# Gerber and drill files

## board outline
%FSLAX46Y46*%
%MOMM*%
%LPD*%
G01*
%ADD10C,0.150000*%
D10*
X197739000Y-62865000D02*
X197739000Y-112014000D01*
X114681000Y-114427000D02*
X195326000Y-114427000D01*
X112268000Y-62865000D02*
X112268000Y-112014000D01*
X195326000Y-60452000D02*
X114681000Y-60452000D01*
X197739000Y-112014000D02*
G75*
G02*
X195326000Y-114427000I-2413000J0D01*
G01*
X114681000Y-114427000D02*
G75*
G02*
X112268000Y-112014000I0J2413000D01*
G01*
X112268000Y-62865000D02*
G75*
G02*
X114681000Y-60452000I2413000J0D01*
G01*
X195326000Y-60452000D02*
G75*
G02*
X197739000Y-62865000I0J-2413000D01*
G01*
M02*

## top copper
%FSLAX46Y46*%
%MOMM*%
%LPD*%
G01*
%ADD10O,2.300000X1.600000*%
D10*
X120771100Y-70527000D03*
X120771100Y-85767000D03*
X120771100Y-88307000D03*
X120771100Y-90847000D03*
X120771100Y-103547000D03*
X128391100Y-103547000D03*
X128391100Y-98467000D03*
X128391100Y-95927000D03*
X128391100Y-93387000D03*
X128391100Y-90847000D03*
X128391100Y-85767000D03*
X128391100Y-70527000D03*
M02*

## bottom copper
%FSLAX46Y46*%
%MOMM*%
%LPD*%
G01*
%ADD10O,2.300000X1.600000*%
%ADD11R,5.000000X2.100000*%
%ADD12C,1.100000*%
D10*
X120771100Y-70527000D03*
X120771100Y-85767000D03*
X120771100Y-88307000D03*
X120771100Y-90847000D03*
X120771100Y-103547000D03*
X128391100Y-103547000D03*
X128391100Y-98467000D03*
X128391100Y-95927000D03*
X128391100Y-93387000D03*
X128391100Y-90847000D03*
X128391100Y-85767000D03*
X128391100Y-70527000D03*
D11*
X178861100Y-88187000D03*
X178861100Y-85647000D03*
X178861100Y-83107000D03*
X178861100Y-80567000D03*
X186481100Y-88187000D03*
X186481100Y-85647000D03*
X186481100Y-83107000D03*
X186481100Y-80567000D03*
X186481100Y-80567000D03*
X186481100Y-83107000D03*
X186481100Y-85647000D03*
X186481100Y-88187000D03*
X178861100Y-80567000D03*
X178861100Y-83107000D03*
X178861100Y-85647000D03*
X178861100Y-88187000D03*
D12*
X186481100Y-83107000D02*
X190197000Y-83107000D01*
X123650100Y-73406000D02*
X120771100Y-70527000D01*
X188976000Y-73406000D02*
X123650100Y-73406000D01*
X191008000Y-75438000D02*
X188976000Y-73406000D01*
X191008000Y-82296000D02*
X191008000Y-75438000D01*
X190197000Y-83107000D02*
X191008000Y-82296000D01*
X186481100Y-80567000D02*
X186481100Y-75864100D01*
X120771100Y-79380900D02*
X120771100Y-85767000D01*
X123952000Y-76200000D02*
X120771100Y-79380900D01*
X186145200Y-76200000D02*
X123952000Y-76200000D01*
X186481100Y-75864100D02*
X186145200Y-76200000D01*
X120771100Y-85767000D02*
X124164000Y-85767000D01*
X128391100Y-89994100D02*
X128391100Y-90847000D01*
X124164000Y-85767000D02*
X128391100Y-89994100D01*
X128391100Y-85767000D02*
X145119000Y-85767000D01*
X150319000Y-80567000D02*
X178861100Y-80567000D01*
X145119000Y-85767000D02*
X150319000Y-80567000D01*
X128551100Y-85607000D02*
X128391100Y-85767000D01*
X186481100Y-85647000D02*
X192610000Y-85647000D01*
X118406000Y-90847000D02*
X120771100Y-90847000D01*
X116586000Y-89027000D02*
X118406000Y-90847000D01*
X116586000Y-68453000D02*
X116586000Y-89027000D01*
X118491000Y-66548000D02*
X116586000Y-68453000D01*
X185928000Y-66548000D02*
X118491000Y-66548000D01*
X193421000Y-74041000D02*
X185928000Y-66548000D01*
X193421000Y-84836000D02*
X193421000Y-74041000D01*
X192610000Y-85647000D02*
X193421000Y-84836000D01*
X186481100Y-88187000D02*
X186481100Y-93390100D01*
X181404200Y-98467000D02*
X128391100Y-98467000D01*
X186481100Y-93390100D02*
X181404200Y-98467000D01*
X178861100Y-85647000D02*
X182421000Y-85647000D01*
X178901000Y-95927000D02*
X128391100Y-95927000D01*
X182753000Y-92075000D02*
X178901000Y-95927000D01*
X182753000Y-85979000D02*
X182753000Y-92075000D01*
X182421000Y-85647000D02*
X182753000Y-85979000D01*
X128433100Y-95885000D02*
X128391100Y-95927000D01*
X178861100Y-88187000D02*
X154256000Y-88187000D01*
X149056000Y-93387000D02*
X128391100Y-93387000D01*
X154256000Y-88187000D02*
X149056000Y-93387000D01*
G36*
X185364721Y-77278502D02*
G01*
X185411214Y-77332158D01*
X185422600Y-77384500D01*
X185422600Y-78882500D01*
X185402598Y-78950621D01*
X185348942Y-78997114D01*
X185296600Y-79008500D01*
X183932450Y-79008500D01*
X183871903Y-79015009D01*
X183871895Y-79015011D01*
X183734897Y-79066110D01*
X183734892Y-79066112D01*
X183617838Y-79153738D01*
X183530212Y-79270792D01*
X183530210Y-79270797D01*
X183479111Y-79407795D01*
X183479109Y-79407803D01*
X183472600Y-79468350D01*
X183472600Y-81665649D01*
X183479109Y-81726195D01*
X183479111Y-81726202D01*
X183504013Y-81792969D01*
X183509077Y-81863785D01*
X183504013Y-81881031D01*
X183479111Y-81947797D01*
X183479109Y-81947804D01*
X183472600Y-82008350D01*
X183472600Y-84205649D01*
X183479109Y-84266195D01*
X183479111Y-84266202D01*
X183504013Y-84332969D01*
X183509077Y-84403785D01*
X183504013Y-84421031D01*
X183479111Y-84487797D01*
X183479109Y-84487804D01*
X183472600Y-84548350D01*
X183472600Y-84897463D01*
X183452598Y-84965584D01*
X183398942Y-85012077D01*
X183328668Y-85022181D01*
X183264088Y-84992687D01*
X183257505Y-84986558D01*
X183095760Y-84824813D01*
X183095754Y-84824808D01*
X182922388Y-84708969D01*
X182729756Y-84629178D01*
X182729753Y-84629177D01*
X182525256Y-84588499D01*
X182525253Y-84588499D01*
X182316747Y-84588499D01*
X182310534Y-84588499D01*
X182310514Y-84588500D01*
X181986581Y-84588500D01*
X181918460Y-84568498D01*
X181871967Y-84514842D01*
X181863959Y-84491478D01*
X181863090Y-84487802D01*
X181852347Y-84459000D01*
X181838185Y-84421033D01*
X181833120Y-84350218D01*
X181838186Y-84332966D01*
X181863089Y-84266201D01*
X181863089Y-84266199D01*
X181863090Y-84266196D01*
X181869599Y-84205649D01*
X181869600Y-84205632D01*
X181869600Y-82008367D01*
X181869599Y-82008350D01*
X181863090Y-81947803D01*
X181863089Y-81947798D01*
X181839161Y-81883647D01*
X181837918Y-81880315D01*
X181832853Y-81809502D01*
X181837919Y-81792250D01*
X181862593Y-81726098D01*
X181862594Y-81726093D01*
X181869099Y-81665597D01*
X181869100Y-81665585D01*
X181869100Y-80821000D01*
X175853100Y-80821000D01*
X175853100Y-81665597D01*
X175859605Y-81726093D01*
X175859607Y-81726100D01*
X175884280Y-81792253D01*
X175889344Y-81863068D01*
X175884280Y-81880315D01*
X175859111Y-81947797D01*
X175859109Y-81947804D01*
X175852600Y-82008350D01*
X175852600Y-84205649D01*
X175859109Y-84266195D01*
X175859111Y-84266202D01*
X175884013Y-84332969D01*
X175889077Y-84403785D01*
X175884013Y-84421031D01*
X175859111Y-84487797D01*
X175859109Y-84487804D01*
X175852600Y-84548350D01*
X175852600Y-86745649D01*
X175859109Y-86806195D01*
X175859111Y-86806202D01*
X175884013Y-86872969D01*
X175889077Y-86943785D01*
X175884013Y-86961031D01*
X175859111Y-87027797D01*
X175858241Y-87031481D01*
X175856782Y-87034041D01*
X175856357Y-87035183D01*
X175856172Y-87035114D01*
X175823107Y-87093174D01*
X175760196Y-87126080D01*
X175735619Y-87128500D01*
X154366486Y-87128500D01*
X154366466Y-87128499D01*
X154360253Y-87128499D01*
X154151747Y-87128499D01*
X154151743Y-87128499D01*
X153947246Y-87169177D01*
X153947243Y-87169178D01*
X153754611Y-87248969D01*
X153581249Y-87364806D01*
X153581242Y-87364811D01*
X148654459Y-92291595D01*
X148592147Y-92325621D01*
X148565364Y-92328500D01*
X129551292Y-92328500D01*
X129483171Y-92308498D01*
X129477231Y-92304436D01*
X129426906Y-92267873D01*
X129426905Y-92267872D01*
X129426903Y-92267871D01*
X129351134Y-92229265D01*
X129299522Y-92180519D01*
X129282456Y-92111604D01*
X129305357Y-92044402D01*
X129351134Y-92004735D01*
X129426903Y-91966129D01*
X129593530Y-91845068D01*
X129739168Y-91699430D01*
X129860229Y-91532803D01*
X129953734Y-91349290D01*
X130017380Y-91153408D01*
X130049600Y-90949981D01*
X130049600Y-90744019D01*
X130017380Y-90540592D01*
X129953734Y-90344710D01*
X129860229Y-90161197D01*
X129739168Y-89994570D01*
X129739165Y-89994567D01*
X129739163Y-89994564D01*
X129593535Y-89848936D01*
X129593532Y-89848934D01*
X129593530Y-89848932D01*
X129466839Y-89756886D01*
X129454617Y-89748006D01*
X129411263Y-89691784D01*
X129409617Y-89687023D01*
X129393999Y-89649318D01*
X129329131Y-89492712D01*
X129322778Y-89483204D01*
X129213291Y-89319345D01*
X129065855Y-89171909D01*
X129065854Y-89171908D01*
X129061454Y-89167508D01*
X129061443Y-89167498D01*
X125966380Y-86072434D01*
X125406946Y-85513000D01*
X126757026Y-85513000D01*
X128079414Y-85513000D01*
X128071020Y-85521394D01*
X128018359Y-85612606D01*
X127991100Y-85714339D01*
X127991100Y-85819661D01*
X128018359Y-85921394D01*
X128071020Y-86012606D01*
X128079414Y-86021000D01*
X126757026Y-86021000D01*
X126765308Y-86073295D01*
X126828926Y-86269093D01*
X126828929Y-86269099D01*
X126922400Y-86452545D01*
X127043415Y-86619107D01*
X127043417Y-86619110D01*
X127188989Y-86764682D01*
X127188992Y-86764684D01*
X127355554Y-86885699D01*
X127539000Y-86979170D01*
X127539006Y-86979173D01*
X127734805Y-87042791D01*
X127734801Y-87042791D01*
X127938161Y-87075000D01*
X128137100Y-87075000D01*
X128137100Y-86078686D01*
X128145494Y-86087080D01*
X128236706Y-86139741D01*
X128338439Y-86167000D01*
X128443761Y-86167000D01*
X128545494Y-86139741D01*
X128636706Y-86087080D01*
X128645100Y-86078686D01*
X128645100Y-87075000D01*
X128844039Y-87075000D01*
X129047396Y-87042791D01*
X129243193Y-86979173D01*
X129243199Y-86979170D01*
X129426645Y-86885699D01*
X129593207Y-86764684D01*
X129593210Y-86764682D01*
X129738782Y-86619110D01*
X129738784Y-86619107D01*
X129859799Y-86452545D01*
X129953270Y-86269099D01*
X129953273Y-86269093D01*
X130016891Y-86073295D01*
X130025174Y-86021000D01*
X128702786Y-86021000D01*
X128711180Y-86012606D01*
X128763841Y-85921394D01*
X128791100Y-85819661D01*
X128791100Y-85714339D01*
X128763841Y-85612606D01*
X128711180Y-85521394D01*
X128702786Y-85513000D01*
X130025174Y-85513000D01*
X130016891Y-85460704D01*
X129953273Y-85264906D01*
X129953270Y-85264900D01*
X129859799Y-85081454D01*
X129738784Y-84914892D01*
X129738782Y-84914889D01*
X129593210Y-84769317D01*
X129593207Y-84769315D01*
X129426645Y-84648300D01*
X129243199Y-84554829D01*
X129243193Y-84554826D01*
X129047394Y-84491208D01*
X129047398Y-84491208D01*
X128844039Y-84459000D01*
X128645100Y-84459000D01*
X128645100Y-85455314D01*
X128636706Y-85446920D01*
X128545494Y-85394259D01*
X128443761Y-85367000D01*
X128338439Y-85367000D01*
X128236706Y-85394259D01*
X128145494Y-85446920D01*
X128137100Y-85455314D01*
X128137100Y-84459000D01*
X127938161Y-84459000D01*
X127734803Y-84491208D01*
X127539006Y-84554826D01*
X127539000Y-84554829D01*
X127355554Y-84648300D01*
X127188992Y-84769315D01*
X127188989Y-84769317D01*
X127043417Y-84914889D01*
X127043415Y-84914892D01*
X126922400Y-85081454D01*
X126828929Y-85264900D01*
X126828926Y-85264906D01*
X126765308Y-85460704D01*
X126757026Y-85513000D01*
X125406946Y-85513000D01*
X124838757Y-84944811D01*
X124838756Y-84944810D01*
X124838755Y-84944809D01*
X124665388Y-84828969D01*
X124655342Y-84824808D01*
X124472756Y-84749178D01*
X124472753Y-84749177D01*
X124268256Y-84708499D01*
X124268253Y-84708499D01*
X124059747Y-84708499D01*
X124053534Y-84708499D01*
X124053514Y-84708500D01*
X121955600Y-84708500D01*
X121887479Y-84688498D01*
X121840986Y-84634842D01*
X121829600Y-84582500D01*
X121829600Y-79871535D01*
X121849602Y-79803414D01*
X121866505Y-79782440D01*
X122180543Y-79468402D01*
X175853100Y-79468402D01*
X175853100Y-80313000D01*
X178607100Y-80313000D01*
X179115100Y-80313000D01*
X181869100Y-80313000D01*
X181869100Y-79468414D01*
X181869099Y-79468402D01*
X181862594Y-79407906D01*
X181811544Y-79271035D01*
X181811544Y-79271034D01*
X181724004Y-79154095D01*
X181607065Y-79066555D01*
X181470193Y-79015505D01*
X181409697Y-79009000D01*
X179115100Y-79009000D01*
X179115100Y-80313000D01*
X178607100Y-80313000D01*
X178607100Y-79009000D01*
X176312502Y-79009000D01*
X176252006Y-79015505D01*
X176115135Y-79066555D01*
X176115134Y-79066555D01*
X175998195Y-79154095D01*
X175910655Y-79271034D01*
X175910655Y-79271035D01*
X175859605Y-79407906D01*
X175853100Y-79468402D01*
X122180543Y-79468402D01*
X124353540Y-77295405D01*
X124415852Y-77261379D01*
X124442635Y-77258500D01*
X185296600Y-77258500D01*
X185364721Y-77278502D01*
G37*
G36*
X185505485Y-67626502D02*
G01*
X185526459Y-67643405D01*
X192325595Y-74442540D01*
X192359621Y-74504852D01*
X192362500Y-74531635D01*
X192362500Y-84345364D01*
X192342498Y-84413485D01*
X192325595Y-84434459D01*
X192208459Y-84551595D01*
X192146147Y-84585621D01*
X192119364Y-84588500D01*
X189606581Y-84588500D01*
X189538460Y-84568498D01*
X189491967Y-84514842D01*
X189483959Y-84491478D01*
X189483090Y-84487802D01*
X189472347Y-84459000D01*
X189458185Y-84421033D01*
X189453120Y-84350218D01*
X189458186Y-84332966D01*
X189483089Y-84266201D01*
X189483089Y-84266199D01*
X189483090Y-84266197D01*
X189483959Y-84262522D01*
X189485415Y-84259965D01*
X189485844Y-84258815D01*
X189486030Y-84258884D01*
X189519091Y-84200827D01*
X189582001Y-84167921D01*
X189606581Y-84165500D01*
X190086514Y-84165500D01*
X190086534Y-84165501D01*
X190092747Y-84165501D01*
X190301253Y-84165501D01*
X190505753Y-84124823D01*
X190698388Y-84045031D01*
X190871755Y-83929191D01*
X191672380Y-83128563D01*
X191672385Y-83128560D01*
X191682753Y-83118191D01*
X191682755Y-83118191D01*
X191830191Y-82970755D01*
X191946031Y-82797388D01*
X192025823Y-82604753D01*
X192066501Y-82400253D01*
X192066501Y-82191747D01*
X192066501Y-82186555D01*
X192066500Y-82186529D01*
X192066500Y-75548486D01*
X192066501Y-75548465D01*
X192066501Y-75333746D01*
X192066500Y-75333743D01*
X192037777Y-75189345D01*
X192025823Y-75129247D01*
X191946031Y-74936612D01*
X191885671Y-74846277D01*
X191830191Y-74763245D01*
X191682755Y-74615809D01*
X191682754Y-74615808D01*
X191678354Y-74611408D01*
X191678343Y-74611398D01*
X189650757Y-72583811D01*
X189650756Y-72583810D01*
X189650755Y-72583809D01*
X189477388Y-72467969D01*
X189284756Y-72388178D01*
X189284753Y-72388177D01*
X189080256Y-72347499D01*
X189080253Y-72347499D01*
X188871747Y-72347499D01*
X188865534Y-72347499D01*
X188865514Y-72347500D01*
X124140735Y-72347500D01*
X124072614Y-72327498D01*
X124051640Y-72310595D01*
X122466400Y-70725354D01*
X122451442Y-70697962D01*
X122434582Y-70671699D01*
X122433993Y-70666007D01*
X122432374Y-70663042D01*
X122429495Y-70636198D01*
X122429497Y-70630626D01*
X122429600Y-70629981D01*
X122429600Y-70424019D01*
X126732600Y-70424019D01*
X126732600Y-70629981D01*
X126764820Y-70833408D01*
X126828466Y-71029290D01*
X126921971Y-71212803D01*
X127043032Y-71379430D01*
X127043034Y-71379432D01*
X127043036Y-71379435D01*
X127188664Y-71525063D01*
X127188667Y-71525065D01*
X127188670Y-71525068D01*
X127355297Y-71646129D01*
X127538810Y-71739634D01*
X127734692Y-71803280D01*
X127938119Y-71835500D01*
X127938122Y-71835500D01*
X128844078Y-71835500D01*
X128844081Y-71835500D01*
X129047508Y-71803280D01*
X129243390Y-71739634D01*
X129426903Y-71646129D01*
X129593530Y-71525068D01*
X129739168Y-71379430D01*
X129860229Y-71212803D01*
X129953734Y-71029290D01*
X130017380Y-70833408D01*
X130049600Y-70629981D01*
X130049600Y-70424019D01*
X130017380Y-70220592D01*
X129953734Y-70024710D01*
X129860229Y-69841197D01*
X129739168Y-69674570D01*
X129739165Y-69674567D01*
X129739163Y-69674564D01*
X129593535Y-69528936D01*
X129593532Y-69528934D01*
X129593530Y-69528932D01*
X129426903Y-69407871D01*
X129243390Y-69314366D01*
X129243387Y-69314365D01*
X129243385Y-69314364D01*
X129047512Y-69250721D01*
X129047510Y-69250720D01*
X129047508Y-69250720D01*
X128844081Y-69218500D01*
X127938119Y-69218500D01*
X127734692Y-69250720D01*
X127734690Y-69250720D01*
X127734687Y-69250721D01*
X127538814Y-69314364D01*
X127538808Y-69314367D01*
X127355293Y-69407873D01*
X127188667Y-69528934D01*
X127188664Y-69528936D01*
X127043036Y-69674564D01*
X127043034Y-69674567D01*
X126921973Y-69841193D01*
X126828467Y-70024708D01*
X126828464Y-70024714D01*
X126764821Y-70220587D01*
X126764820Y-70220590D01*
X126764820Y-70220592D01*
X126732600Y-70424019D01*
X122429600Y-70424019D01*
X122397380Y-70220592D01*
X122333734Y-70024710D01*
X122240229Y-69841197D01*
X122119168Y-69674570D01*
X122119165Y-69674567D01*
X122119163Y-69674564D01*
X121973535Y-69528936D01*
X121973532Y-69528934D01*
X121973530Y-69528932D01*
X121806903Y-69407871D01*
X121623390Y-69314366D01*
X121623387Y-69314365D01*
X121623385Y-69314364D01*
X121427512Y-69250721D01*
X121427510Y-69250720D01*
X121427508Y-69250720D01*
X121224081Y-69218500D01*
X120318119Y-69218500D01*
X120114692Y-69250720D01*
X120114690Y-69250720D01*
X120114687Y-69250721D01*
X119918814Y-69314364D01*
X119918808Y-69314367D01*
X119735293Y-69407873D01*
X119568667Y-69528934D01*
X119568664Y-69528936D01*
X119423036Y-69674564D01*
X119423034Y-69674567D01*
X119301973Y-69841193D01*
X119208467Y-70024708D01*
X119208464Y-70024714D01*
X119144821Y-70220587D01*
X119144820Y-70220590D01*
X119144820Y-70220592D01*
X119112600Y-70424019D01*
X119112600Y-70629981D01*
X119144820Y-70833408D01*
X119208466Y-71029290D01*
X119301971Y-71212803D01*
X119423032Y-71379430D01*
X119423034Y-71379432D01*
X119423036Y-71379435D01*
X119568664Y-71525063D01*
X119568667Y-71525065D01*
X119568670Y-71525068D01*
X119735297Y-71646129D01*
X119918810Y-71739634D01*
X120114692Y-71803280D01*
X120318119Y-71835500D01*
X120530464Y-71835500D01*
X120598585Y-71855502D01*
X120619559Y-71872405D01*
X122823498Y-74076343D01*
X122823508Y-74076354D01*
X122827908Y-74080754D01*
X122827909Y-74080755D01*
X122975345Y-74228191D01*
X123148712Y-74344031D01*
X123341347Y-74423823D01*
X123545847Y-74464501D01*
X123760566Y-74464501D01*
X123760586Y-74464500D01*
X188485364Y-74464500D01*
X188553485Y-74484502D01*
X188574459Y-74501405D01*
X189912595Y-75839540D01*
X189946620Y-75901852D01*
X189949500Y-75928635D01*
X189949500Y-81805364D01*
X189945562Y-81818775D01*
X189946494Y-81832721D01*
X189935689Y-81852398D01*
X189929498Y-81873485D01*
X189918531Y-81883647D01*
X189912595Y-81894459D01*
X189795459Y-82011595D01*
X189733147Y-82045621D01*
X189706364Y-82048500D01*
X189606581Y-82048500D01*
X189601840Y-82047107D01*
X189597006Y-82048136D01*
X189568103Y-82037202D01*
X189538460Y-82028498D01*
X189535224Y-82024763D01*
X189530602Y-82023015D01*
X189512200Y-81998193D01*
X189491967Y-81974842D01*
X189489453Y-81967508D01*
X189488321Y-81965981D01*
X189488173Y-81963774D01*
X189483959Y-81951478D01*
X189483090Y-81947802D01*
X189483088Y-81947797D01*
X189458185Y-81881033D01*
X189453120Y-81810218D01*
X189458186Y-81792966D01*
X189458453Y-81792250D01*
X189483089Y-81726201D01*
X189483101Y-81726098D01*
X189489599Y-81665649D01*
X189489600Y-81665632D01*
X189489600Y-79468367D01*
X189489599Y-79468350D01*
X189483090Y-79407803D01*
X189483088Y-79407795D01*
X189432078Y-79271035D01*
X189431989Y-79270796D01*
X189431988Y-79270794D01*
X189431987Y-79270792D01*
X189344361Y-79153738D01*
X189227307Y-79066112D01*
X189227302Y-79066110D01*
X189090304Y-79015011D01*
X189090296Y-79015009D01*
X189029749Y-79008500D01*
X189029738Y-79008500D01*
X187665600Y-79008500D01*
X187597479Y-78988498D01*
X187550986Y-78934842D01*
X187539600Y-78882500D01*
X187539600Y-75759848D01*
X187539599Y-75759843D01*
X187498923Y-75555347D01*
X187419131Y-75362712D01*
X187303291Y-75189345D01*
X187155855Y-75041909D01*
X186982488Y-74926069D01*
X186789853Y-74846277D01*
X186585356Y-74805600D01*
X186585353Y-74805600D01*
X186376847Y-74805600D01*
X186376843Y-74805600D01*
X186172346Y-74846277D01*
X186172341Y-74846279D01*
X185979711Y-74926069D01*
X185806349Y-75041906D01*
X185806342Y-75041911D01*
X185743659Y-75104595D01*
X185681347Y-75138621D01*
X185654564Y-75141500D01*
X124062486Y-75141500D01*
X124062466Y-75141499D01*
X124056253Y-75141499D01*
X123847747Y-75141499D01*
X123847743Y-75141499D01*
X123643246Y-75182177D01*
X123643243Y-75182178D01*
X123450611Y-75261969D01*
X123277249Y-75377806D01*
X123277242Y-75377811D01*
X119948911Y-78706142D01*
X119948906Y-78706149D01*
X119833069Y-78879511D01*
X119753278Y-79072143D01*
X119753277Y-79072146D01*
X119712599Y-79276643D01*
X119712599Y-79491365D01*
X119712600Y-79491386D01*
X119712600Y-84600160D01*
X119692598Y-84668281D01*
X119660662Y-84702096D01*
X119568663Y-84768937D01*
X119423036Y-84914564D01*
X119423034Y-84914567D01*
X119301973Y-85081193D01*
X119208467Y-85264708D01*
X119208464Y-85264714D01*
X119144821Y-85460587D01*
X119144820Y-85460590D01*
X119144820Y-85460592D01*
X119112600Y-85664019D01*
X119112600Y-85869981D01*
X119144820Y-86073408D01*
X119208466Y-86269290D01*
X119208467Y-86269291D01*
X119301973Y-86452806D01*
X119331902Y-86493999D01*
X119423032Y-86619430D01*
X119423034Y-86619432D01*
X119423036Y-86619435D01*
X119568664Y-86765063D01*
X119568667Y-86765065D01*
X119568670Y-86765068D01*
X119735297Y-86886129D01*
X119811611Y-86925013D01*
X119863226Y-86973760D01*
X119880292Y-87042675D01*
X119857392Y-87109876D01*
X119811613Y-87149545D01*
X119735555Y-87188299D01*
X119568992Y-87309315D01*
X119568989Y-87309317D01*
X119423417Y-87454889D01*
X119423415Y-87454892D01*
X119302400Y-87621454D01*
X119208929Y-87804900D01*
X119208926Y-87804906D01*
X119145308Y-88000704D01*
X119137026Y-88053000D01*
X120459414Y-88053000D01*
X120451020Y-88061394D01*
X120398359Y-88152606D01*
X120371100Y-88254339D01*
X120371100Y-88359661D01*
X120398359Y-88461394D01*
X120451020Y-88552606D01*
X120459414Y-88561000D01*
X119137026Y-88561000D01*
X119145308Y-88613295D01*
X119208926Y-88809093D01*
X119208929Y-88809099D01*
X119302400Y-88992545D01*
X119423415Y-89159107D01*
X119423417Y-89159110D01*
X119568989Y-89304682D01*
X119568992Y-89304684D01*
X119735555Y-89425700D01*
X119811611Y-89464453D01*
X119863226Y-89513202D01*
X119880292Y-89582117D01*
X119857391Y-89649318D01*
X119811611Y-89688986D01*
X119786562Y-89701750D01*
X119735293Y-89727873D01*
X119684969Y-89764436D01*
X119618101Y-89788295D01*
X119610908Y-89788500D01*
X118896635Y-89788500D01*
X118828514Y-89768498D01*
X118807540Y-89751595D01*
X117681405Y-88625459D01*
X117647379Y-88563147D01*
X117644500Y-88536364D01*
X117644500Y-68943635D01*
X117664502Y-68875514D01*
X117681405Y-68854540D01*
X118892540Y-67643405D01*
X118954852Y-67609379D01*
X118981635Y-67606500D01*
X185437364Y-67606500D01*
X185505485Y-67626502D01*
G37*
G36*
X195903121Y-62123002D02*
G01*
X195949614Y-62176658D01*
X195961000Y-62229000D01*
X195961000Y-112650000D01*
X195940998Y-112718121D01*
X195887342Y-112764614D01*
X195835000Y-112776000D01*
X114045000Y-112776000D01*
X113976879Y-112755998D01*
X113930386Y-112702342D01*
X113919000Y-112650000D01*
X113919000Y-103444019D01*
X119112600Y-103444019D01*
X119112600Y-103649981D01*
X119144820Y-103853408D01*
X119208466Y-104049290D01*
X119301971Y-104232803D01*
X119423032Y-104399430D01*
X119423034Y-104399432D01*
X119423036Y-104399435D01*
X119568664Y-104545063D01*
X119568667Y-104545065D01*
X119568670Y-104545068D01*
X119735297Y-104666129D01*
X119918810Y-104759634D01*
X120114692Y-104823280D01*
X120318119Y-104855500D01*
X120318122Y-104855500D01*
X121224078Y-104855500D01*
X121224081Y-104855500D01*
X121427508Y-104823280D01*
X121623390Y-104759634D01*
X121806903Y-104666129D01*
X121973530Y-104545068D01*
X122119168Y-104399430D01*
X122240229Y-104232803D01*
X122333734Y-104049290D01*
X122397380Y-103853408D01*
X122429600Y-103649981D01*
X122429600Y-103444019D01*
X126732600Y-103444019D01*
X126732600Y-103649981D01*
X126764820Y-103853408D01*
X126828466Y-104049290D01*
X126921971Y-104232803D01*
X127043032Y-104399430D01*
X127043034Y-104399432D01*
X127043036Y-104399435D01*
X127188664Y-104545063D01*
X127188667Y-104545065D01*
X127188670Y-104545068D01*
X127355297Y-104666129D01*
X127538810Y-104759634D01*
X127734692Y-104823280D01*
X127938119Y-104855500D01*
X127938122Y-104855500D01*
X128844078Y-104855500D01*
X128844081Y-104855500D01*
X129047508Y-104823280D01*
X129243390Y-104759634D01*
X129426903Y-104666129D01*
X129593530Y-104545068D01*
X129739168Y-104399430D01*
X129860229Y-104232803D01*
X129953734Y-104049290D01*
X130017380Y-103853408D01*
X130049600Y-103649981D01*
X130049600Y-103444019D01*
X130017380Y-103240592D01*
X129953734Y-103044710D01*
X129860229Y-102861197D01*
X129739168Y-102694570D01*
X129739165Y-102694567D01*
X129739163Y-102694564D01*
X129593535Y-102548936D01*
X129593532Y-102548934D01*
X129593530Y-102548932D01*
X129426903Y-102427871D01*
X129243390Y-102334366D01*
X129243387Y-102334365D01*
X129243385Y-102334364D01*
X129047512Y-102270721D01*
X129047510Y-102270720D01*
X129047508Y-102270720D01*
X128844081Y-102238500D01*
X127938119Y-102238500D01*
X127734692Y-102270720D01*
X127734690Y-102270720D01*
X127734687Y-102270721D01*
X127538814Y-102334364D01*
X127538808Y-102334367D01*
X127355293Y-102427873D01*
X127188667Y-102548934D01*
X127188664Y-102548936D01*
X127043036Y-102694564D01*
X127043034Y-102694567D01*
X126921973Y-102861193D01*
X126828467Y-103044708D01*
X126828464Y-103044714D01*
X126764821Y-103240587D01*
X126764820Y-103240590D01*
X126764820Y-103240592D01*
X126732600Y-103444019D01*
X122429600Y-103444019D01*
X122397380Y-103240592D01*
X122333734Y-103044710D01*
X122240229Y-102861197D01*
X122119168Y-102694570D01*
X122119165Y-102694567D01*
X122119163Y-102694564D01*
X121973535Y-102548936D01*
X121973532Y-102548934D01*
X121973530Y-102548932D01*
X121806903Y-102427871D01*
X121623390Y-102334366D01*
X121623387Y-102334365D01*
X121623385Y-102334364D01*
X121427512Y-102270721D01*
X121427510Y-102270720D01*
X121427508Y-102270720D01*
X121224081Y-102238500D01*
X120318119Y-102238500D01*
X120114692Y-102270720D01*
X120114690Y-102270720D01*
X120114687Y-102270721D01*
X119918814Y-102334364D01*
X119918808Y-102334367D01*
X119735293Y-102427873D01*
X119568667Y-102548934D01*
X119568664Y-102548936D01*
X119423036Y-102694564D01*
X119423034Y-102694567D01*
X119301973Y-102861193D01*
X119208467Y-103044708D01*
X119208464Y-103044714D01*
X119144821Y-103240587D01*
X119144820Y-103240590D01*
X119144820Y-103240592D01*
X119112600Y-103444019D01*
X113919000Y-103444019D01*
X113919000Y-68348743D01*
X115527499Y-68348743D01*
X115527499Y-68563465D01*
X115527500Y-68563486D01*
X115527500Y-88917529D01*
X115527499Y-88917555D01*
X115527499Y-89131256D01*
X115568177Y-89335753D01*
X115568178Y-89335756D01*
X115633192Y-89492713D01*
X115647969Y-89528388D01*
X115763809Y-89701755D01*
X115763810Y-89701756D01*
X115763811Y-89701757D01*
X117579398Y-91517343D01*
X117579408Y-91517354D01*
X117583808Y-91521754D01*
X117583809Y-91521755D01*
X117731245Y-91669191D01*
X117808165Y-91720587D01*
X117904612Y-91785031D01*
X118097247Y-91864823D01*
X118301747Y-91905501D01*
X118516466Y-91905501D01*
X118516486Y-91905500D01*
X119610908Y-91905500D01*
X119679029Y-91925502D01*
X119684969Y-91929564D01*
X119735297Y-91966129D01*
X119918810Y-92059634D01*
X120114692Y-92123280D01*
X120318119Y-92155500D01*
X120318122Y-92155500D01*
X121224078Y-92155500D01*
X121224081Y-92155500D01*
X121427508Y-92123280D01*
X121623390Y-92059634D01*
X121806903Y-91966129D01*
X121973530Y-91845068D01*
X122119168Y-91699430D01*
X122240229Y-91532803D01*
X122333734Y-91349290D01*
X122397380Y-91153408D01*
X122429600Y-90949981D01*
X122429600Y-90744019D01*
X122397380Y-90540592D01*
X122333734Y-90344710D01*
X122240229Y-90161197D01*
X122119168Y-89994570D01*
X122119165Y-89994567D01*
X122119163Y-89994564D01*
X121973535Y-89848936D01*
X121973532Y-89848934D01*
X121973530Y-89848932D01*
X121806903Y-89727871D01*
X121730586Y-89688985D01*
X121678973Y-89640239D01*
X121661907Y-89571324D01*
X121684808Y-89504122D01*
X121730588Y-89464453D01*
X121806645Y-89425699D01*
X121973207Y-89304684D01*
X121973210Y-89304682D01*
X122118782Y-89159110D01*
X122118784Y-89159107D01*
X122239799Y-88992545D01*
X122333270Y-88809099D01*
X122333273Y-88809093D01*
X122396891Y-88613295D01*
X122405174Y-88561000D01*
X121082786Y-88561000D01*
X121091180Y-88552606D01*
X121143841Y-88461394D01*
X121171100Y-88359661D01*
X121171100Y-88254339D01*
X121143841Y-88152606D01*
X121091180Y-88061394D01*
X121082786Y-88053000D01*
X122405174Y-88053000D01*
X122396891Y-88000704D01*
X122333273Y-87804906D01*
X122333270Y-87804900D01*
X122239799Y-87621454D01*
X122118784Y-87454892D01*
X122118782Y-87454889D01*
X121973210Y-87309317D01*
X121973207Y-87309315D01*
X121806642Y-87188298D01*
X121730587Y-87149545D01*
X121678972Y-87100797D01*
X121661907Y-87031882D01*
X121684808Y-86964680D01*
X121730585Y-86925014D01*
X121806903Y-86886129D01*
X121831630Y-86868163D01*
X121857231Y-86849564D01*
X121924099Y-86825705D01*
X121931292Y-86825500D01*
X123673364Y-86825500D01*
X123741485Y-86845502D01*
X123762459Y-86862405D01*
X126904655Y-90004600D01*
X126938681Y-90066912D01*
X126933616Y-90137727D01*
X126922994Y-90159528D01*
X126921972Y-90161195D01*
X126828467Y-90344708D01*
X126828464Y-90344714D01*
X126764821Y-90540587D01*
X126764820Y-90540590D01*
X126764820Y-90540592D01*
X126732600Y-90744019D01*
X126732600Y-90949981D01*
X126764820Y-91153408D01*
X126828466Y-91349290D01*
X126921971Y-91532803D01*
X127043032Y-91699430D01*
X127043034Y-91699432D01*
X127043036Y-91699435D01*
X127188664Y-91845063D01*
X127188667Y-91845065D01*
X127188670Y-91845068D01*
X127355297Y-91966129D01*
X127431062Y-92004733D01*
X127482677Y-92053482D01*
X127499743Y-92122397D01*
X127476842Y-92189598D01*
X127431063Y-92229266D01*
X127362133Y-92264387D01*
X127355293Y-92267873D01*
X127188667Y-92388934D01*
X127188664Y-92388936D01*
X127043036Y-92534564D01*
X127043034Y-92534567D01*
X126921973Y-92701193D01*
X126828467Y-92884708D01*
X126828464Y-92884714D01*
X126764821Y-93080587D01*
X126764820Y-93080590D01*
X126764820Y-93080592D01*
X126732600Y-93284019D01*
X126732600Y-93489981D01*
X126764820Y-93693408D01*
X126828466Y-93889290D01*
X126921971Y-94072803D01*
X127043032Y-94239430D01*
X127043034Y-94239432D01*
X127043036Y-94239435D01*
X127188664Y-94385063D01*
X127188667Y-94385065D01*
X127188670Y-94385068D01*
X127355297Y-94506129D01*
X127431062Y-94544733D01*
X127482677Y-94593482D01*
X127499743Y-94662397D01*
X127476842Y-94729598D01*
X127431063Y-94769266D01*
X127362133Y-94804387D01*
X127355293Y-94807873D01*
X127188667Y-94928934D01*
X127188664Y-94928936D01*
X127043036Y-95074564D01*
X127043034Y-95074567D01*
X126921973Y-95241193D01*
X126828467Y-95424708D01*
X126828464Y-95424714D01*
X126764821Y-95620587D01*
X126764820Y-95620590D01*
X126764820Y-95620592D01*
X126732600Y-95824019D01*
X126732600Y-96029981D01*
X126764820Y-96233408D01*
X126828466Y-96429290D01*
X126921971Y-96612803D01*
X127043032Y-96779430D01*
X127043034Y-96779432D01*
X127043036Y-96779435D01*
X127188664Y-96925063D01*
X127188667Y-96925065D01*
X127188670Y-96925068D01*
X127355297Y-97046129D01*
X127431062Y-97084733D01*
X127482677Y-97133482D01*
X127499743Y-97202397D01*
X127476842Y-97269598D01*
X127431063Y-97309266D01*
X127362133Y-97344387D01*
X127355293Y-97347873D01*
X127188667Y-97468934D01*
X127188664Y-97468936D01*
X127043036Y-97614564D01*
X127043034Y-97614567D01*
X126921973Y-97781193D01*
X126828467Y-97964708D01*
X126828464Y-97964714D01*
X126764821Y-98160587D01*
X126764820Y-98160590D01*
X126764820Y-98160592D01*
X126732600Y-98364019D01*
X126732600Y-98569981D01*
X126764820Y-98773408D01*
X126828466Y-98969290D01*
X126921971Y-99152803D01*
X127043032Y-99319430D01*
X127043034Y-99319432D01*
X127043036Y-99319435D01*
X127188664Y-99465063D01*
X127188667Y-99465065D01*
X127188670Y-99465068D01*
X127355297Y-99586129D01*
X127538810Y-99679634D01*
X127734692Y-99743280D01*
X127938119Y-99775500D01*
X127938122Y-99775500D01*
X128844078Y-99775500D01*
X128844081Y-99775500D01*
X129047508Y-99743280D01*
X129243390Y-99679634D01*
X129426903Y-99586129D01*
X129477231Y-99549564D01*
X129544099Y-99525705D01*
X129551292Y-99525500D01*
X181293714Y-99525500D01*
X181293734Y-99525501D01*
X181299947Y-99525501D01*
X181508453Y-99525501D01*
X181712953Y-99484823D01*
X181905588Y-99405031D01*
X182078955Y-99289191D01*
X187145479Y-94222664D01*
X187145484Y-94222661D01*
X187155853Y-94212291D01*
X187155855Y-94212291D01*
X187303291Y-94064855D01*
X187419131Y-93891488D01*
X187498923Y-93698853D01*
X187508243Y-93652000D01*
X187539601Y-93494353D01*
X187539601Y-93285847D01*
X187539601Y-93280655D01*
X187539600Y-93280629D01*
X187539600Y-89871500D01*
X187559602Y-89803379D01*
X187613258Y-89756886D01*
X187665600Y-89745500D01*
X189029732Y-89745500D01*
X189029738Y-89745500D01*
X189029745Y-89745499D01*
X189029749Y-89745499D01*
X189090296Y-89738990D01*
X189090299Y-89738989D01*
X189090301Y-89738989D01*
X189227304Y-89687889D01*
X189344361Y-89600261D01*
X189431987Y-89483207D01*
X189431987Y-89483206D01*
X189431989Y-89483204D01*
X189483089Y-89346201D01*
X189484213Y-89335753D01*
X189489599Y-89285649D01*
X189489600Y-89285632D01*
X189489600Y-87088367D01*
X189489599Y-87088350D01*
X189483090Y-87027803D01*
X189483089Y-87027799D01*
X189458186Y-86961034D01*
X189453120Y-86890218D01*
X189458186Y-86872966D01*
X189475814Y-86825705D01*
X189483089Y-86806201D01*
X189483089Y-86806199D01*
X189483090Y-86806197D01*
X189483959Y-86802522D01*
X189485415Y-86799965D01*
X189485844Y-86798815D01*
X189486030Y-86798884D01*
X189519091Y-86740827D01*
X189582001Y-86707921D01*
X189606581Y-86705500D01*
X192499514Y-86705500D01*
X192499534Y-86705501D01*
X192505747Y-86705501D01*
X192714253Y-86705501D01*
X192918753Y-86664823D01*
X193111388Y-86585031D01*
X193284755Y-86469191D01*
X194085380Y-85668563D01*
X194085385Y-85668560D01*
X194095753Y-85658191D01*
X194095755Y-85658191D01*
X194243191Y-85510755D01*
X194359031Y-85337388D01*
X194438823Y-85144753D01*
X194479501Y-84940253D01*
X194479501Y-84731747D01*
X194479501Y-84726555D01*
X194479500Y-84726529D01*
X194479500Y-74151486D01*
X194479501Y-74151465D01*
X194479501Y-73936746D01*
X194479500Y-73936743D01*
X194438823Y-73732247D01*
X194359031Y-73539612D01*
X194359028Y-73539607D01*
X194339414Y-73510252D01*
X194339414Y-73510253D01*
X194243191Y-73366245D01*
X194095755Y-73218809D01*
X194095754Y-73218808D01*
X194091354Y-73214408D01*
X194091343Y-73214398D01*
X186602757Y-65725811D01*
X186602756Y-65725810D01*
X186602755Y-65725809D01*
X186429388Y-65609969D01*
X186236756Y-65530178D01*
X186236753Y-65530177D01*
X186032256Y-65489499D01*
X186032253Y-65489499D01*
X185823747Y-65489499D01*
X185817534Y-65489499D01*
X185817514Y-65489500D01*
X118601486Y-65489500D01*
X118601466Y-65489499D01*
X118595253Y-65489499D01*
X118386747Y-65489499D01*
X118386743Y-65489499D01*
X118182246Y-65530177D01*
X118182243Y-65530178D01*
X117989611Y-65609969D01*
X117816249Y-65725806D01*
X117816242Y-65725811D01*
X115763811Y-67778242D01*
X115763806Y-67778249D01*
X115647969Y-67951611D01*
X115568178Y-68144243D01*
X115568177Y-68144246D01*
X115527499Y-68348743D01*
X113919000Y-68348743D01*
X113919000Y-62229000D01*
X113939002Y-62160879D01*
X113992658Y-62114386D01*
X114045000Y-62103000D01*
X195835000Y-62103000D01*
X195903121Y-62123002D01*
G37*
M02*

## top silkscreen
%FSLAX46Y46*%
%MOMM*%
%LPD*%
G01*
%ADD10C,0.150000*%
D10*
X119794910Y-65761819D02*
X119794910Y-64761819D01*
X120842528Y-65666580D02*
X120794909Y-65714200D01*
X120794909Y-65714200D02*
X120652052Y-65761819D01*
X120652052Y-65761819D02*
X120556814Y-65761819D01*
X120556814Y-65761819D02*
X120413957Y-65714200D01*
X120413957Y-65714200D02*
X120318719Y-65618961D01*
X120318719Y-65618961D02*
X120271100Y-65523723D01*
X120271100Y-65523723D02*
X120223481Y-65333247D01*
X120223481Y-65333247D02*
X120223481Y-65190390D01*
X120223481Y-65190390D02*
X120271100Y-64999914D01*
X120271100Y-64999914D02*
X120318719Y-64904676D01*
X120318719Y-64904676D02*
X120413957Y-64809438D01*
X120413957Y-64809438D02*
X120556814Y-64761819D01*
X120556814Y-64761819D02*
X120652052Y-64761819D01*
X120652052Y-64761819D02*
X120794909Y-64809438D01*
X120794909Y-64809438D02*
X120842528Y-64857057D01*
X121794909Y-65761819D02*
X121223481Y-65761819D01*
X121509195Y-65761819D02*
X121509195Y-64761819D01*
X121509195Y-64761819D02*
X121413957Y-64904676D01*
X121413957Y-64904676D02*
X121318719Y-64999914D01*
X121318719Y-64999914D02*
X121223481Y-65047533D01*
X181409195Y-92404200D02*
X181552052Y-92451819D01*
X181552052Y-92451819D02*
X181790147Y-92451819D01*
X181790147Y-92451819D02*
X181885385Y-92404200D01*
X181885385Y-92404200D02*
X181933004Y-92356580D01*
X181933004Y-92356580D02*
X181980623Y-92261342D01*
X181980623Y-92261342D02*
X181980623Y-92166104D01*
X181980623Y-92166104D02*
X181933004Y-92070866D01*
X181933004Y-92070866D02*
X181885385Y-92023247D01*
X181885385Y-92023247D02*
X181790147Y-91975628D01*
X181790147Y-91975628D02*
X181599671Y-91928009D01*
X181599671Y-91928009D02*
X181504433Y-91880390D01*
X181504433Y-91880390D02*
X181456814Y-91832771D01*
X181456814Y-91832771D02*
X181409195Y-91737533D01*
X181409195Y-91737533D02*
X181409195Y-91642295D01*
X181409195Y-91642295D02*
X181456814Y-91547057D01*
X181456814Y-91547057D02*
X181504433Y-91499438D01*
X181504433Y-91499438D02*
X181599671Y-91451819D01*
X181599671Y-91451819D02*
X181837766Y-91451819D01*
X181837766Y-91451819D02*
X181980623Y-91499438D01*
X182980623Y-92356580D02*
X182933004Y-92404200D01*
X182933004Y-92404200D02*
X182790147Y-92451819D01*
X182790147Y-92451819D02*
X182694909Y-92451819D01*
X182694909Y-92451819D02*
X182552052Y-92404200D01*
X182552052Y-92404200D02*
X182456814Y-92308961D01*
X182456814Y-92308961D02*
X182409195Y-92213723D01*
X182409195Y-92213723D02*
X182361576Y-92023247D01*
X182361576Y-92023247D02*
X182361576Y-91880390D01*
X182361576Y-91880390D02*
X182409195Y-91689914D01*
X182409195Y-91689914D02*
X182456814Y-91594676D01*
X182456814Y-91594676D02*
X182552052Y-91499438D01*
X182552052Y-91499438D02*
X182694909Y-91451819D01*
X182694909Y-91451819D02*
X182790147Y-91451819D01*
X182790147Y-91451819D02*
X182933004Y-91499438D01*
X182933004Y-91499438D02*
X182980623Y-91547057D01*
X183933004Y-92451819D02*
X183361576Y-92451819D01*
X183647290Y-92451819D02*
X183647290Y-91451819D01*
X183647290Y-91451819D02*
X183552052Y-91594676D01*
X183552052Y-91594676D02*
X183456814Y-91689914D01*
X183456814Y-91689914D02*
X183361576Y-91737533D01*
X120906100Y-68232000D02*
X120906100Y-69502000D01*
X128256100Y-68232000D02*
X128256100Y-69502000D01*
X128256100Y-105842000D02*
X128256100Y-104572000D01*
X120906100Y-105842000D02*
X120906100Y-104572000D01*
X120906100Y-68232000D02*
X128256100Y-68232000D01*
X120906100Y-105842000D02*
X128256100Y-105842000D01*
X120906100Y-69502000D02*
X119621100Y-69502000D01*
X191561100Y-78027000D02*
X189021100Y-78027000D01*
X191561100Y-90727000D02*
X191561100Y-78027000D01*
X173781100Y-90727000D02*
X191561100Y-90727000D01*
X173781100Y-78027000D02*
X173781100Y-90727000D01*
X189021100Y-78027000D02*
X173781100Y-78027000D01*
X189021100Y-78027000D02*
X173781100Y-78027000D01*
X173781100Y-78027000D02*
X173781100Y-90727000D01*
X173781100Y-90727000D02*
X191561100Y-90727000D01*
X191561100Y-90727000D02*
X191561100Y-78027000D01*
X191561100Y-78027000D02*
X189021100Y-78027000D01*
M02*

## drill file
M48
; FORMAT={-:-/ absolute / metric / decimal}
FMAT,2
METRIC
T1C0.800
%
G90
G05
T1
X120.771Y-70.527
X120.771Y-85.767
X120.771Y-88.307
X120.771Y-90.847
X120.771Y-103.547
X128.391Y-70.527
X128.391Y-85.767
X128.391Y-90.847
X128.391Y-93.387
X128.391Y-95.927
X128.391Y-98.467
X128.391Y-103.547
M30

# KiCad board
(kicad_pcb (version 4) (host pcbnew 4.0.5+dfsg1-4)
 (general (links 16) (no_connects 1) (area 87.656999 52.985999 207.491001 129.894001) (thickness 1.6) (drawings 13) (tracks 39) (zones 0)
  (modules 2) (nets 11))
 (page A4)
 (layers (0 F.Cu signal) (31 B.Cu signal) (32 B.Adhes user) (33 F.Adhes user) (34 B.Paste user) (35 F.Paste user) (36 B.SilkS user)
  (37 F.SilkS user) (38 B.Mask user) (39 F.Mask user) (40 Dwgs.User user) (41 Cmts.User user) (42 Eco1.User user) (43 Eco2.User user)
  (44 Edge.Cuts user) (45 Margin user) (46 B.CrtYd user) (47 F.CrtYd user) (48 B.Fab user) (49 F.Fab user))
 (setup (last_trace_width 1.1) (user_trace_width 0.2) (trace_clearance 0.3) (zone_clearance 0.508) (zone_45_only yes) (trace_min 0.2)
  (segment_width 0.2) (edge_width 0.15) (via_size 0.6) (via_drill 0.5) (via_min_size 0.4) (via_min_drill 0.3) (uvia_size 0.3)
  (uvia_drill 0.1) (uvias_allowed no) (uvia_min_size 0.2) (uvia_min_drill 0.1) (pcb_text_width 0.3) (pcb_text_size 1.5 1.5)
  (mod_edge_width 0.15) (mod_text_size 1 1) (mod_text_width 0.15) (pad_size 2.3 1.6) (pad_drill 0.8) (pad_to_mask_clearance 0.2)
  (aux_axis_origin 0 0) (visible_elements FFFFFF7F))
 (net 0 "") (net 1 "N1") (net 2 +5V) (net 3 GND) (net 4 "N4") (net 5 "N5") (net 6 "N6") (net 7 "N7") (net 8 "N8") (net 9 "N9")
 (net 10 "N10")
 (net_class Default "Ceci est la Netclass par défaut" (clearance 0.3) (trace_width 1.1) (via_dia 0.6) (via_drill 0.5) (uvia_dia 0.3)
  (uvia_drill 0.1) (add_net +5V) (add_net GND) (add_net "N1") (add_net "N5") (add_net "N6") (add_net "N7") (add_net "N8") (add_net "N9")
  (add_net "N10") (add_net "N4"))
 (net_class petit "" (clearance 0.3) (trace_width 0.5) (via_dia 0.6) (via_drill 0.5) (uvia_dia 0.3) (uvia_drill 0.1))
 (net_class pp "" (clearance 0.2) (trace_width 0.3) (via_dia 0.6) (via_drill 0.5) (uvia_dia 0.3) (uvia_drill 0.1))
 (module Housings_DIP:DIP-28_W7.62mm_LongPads (layer F.Cu) (at 120.7711 70.527)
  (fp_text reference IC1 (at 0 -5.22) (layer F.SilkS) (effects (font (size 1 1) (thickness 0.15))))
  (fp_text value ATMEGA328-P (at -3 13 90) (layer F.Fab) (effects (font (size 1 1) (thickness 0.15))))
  (fp_line (start 0.135 -2.295) (end 0.135 -1.025) (layer F.SilkS) (width 0.15))
  (fp_line (start 7.485 -2.295) (end 7.485 -1.025) (layer F.SilkS) (width 0.15))
  (fp_line (start 7.485 35.315) (end 7.485 34.045) (layer F.SilkS) (width 0.15))
  (fp_line (start 0.135 35.315) (end 0.135 34.045) (layer F.SilkS) (width 0.15))
  (fp_line (start 0.135 -2.295) (end 7.485 -2.295) (layer F.SilkS) (width 0.15))
  (fp_line (start 0.135 35.315) (end 7.485 35.315) (layer F.SilkS) (width 0.15))
  (fp_line (start 0.135 -1.025) (end -1.15 -1.025) (layer F.SilkS) (width 0.15))
  (pad 1 thru_hole oval (at 0 0) (size 2.3 1.6) (drill 0.8) (layers *.Cu *.Mask) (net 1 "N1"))
  (pad 7 thru_hole oval (at 0 15.24) (size 2.3 1.6) (drill 0.8) (layers *.Cu *.Mask) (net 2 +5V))
  (pad 8 thru_hole oval (at 0 17.78) (size 2.3 1.6) (drill 0.8) (layers *.Cu *.Mask) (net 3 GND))
  (pad 9 thru_hole oval (at 0 20.32) (size 2.3 1.6) (drill 0.8) (layers *.Cu *.Mask) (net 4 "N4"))
  (pad 14 thru_hole oval (at 0 33.02) (size 2.3 1.6) (drill 0.8) (layers *.Cu *.Mask) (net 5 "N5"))
  (pad 15 thru_hole oval (at 7.62 33.02) (size 2.3 1.6) (drill 0.8) (layers *.Cu *.Mask) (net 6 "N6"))
  (pad 17 thru_hole oval (at 7.62 27.94) (size 2.3 1.6) (drill 0.8) (layers *.Cu *.Mask) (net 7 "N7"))
  (pad 18 thru_hole oval (at 7.62 25.4) (size 2.3 1.6) (drill 0.8) (layers *.Cu *.Mask) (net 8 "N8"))
  (pad 19 thru_hole oval (at 7.62 22.86) (size 2.3 1.6) (drill 0.8) (layers *.Cu *.Mask) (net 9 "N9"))
  (pad 20 thru_hole oval (at 7.62 20.32) (size 2.3 1.6) (drill 0.8) (layers *.Cu *.Mask) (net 2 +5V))
  (pad 22 thru_hole oval (at 7.62 15.24) (size 2.3 1.6) (drill 0.8) (layers *.Cu *.Mask) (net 3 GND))
  (pad 28 thru_hole oval (at 7.62 0) (size 2.3 1.6) (drill 0.8) (layers *.Cu *.Mask) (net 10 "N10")))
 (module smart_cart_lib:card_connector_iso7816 (layer F.Cu) (at 182.6711 90.727)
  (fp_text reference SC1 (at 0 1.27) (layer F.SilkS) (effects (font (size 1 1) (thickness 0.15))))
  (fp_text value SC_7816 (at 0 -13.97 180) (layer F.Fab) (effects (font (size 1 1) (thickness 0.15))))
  (fp_line (start 8.89 -12.7) (end 6.35 -12.7) (layer F.SilkS) (width 0.15))
  (fp_line (start 8.89 0) (end 8.89 -12.7) (layer F.SilkS) (width 0.15))
  (fp_line (start -8.89 0) (end 8.89 0) (layer F.SilkS) (width 0.15))
  (fp_line (start -8.89 -12.7) (end -8.89 0) (layer F.SilkS) (width 0.15))
  (fp_line (start 6.35 -12.7) (end -8.89 -12.7) (layer F.SilkS) (width 0.15))
  (fp_line (start 6.35 -12.7) (end -8.89 -12.7) (layer F.SilkS) (width 0.15))
  (fp_line (start -8.89 -12.7) (end -8.89 0) (layer F.SilkS) (width 0.15))
  (fp_line (start -8.89 0) (end 8.89 0) (layer F.SilkS) (width 0.15))
  (fp_line (start 8.89 0) (end 8.89 -12.7) (layer F.SilkS) (width 0.15))
  (fp_line (start 8.89 -12.7) (end 6.35 -12.7) (layer F.SilkS) (width 0.15))
  (pad c8 connect rect (at -3.81 -2.54) (size 5 2.1) (layers B.Cu F.Mask) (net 9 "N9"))
  (pad c7 connect rect (at -3.81 -5.08) (size 5 2.1) (layers B.Cu F.Mask) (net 8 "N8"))
  (pad c6 connect rect (at -3.81 -7.62) (size 5 2.1) (layers B.Cu F.Mask))
  (pad c5 connect rect (at -3.81 -10.16) (size 5 2.1) (layers B.Cu F.Mask) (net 3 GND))
  (pad c4 connect rect (at 3.81 -2.54) (size 5 2.1) (layers B.Cu F.Mask) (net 7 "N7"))
  (pad c3 connect rect (at 3.81 -5.08) (size 5 2.1) (layers B.Cu F.Mask) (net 4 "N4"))
  (pad c2 connect rect (at 3.81 -7.62) (size 5 2.1) (layers B.Cu F.Mask) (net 1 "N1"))
  (pad c1 connect rect (at 3.81 -10.16) (size 5 2.1) (layers B.Cu F.Mask) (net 2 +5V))
  (pad c1 connect rect (at 3.81 -10.16) (size 5 2.1) (layers B.Cu F.Mask) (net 2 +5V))
  (pad c2 connect rect (at 3.81 -7.62) (size 5 2.1) (layers B.Cu F.Mask) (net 1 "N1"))
  (pad c3 connect rect (at 3.81 -5.08) (size 5 2.1) (layers B.Cu F.Mask) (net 4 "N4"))
  (pad c4 connect rect (at 3.81 -2.54) (size 5 2.1) (layers B.Cu F.Mask) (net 7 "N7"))
  (pad c5 connect rect (at -3.81 -10.16) (size 5 2.1) (layers B.Cu F.Mask) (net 3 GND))
  (pad c6 connect rect (at -3.81 -7.62) (size 5 2.1) (layers B.Cu F.Mask))
  (pad c7 connect rect (at -3.81 -5.08) (size 5 2.1) (layers B.Cu F.Mask) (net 8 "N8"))
  (pad c8 connect rect (at -3.81 -2.54) (size 5 2.1) (layers B.Cu F.Mask) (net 9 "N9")))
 (gr_line (start 197.739 62.865) (end 197.739 112.014) (angle 90) (layer Edge.Cuts) (width 0.15))
 (gr_line (start 114.681 114.427) (end 195.326 114.427) (angle 90) (layer Edge.Cuts) (width 0.15))
 (gr_line (start 112.268 62.865) (end 112.268 112.014) (angle 90) (layer Edge.Cuts) (width 0.15))
 (gr_line (start 195.326 60.452) (end 114.681 60.452) (angle 90) (layer Edge.Cuts) (width 0.15))
 (gr_arc (start 195.326 112.014) (end 197.739 112.014) (angle 90) (layer Edge.Cuts) (width 0.15))
 (gr_arc (start 114.681 112.014) (end 114.681 114.427) (angle 90) (layer Edge.Cuts) (width 0.15))
 (gr_arc (start 114.681 62.865) (end 112.268 62.865) (angle 90) (layer Edge.Cuts) (width 0.15))
 (gr_arc (start 195.326 62.865) (end 195.326 60.452) (angle 90) (layer Edge.Cuts) (width 0.15))
 (segment (start 186.4811 83.107) (end 190.197 83.107) (width 1.1) (layer B.Cu) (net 1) (status 400000))
 (segment (start 123.6501 73.406) (end 120.7711 70.527) (width 1.1) (layer B.Cu) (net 1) (status 800000))
 (segment (start 188.976 73.406) (end 123.6501 73.406) (width 1.1) (layer B.Cu) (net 1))
 (segment (start 191.008 75.438) (end 188.976 73.406) (width 1.1) (layer B.Cu) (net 1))
 (segment (start 191.008 82.296) (end 191.008 75.438) (width 1.1) (layer B.Cu) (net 1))
 (segment (start 190.197 83.107) (end 191.008 82.296) (width 1.1) (layer B.Cu) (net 1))
 (segment (start 186.4811 80.567) (end 186.4811 75.8641) (width 1.1) (layer B.Cu) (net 2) (status 400000))
 (segment (start 120.7711 79.3809) (end 120.7711 85.767) (width 1.1) (layer B.Cu) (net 2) (status 800000))
 (segment (start 123.952 76.2) (end 120.7711 79.3809) (width 1.1) (layer B.Cu) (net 2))
 (segment (start 186.1452 76.2) (end 123.952 76.2) (width 1.1) (layer B.Cu) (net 2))
 (segment (start 186.4811 75.8641) (end 186.1452 76.2) (width 1.1) (layer B.Cu) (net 2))
 (segment (start 120.7711 85.767) (end 124.164 85.767) (width 1.1) (layer B.Cu) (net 2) (status 400000))
 (segment (start 128.3911 89.9941) (end 128.3911 90.847) (width 1.1) (layer B.Cu) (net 2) (status 800000))
 (segment (start 124.164 85.767) (end 128.3911 89.9941) (width 1.1) (layer B.Cu) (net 2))
 (segment (start 128.3911 85.767) (end 145.119 85.767) (width 1.1) (layer B.Cu) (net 3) (status 400000))
 (segment (start 150.319 80.567) (end 178.8611 80.567) (width 1.1) (layer B.Cu) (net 3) (status 800000))
 (segment (start 145.119 85.767) (end 150.319 80.567) (width 1.1) (layer B.Cu) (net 3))
 (segment (start 128.5511 85.607) (end 128.3911 85.767) (width 1.1) (layer B.Cu) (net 3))
 (segment (start 186.4811 85.647) (end 192.61 85.647) (width 1.1) (layer B.Cu) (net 4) (status 400000))
 (segment (start 118.406 90.847) (end 120.7711 90.847) (width 1.1) (layer B.Cu) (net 4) (status 800000))
 (segment (start 116.586 89.027) (end 118.406 90.847) (width 1.1) (layer B.Cu) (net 4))
 (segment (start 116.586 68.453) (end 116.586 89.027) (width 1.1) (layer B.Cu) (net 4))
 (segment (start 118.491 66.548) (end 116.586 68.453) (width 1.1) (layer B.Cu) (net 4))
 (segment (start 185.928 66.548) (end 118.491 66.548) (width 1.1) (layer B.Cu) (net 4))
 (segment (start 193.421 74.041) (end 185.928 66.548) (width 1.1) (layer B.Cu) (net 4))
 (segment (start 193.421 84.836) (end 193.421 74.041) (width 1.1) (layer B.Cu) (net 4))
 (segment (start 192.61 85.647) (end 193.421 84.836) (width 1.1) (layer B.Cu) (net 4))
 (segment (start 186.4811 88.187) (end 186.4811 93.3901) (width 1.1) (layer B.Cu) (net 7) (status 400000))
 (segment (start 181.4042 98.467) (end 128.3911 98.467) (width 1.1) (layer B.Cu) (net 7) (status 800000))
 (segment (start 186.4811 93.3901) (end 181.4042 98.467) (width 1.1) (layer B.Cu) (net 7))
 (segment (start 178.8611 85.647) (end 182.421 85.647) (width 1.1) (layer B.Cu) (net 8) (status 400000))
 (segment (start 178.901 95.927) (end 128.3911 95.927) (width 1.1) (layer B.Cu) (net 8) (status 800000))
 (segment (start 182.753 92.075) (end 178.901 95.927) (width 1.1) (layer B.Cu) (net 8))
 (segment (start 182.753 85.979) (end 182.753 92.075) (width 1.1) (layer B.Cu) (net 8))
 (segment (start 182.421 85.647) (end 182.753 85.979) (width 1.1) (layer B.Cu) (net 8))
 (segment (start 128.4331 95.885) (end 128.3911 95.927) (width 1.1) (layer B.Cu) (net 8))
 (segment (start 178.8611 88.187) (end 154.256 88.187) (width 1.1) (layer B.Cu) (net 9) (status 400000))
 (segment (start 149.056 93.387) (end 128.3911 93.387) (width 1.1) (layer B.Cu) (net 9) (status 800000))
 (segment (start 154.256 88.187) (end 149.056 93.387) (width 1.1) (layer B.Cu) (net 9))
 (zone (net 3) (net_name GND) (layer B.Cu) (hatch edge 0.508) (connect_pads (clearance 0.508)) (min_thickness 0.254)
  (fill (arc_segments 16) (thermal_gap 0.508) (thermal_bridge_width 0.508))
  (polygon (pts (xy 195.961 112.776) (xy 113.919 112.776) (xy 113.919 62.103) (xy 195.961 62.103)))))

